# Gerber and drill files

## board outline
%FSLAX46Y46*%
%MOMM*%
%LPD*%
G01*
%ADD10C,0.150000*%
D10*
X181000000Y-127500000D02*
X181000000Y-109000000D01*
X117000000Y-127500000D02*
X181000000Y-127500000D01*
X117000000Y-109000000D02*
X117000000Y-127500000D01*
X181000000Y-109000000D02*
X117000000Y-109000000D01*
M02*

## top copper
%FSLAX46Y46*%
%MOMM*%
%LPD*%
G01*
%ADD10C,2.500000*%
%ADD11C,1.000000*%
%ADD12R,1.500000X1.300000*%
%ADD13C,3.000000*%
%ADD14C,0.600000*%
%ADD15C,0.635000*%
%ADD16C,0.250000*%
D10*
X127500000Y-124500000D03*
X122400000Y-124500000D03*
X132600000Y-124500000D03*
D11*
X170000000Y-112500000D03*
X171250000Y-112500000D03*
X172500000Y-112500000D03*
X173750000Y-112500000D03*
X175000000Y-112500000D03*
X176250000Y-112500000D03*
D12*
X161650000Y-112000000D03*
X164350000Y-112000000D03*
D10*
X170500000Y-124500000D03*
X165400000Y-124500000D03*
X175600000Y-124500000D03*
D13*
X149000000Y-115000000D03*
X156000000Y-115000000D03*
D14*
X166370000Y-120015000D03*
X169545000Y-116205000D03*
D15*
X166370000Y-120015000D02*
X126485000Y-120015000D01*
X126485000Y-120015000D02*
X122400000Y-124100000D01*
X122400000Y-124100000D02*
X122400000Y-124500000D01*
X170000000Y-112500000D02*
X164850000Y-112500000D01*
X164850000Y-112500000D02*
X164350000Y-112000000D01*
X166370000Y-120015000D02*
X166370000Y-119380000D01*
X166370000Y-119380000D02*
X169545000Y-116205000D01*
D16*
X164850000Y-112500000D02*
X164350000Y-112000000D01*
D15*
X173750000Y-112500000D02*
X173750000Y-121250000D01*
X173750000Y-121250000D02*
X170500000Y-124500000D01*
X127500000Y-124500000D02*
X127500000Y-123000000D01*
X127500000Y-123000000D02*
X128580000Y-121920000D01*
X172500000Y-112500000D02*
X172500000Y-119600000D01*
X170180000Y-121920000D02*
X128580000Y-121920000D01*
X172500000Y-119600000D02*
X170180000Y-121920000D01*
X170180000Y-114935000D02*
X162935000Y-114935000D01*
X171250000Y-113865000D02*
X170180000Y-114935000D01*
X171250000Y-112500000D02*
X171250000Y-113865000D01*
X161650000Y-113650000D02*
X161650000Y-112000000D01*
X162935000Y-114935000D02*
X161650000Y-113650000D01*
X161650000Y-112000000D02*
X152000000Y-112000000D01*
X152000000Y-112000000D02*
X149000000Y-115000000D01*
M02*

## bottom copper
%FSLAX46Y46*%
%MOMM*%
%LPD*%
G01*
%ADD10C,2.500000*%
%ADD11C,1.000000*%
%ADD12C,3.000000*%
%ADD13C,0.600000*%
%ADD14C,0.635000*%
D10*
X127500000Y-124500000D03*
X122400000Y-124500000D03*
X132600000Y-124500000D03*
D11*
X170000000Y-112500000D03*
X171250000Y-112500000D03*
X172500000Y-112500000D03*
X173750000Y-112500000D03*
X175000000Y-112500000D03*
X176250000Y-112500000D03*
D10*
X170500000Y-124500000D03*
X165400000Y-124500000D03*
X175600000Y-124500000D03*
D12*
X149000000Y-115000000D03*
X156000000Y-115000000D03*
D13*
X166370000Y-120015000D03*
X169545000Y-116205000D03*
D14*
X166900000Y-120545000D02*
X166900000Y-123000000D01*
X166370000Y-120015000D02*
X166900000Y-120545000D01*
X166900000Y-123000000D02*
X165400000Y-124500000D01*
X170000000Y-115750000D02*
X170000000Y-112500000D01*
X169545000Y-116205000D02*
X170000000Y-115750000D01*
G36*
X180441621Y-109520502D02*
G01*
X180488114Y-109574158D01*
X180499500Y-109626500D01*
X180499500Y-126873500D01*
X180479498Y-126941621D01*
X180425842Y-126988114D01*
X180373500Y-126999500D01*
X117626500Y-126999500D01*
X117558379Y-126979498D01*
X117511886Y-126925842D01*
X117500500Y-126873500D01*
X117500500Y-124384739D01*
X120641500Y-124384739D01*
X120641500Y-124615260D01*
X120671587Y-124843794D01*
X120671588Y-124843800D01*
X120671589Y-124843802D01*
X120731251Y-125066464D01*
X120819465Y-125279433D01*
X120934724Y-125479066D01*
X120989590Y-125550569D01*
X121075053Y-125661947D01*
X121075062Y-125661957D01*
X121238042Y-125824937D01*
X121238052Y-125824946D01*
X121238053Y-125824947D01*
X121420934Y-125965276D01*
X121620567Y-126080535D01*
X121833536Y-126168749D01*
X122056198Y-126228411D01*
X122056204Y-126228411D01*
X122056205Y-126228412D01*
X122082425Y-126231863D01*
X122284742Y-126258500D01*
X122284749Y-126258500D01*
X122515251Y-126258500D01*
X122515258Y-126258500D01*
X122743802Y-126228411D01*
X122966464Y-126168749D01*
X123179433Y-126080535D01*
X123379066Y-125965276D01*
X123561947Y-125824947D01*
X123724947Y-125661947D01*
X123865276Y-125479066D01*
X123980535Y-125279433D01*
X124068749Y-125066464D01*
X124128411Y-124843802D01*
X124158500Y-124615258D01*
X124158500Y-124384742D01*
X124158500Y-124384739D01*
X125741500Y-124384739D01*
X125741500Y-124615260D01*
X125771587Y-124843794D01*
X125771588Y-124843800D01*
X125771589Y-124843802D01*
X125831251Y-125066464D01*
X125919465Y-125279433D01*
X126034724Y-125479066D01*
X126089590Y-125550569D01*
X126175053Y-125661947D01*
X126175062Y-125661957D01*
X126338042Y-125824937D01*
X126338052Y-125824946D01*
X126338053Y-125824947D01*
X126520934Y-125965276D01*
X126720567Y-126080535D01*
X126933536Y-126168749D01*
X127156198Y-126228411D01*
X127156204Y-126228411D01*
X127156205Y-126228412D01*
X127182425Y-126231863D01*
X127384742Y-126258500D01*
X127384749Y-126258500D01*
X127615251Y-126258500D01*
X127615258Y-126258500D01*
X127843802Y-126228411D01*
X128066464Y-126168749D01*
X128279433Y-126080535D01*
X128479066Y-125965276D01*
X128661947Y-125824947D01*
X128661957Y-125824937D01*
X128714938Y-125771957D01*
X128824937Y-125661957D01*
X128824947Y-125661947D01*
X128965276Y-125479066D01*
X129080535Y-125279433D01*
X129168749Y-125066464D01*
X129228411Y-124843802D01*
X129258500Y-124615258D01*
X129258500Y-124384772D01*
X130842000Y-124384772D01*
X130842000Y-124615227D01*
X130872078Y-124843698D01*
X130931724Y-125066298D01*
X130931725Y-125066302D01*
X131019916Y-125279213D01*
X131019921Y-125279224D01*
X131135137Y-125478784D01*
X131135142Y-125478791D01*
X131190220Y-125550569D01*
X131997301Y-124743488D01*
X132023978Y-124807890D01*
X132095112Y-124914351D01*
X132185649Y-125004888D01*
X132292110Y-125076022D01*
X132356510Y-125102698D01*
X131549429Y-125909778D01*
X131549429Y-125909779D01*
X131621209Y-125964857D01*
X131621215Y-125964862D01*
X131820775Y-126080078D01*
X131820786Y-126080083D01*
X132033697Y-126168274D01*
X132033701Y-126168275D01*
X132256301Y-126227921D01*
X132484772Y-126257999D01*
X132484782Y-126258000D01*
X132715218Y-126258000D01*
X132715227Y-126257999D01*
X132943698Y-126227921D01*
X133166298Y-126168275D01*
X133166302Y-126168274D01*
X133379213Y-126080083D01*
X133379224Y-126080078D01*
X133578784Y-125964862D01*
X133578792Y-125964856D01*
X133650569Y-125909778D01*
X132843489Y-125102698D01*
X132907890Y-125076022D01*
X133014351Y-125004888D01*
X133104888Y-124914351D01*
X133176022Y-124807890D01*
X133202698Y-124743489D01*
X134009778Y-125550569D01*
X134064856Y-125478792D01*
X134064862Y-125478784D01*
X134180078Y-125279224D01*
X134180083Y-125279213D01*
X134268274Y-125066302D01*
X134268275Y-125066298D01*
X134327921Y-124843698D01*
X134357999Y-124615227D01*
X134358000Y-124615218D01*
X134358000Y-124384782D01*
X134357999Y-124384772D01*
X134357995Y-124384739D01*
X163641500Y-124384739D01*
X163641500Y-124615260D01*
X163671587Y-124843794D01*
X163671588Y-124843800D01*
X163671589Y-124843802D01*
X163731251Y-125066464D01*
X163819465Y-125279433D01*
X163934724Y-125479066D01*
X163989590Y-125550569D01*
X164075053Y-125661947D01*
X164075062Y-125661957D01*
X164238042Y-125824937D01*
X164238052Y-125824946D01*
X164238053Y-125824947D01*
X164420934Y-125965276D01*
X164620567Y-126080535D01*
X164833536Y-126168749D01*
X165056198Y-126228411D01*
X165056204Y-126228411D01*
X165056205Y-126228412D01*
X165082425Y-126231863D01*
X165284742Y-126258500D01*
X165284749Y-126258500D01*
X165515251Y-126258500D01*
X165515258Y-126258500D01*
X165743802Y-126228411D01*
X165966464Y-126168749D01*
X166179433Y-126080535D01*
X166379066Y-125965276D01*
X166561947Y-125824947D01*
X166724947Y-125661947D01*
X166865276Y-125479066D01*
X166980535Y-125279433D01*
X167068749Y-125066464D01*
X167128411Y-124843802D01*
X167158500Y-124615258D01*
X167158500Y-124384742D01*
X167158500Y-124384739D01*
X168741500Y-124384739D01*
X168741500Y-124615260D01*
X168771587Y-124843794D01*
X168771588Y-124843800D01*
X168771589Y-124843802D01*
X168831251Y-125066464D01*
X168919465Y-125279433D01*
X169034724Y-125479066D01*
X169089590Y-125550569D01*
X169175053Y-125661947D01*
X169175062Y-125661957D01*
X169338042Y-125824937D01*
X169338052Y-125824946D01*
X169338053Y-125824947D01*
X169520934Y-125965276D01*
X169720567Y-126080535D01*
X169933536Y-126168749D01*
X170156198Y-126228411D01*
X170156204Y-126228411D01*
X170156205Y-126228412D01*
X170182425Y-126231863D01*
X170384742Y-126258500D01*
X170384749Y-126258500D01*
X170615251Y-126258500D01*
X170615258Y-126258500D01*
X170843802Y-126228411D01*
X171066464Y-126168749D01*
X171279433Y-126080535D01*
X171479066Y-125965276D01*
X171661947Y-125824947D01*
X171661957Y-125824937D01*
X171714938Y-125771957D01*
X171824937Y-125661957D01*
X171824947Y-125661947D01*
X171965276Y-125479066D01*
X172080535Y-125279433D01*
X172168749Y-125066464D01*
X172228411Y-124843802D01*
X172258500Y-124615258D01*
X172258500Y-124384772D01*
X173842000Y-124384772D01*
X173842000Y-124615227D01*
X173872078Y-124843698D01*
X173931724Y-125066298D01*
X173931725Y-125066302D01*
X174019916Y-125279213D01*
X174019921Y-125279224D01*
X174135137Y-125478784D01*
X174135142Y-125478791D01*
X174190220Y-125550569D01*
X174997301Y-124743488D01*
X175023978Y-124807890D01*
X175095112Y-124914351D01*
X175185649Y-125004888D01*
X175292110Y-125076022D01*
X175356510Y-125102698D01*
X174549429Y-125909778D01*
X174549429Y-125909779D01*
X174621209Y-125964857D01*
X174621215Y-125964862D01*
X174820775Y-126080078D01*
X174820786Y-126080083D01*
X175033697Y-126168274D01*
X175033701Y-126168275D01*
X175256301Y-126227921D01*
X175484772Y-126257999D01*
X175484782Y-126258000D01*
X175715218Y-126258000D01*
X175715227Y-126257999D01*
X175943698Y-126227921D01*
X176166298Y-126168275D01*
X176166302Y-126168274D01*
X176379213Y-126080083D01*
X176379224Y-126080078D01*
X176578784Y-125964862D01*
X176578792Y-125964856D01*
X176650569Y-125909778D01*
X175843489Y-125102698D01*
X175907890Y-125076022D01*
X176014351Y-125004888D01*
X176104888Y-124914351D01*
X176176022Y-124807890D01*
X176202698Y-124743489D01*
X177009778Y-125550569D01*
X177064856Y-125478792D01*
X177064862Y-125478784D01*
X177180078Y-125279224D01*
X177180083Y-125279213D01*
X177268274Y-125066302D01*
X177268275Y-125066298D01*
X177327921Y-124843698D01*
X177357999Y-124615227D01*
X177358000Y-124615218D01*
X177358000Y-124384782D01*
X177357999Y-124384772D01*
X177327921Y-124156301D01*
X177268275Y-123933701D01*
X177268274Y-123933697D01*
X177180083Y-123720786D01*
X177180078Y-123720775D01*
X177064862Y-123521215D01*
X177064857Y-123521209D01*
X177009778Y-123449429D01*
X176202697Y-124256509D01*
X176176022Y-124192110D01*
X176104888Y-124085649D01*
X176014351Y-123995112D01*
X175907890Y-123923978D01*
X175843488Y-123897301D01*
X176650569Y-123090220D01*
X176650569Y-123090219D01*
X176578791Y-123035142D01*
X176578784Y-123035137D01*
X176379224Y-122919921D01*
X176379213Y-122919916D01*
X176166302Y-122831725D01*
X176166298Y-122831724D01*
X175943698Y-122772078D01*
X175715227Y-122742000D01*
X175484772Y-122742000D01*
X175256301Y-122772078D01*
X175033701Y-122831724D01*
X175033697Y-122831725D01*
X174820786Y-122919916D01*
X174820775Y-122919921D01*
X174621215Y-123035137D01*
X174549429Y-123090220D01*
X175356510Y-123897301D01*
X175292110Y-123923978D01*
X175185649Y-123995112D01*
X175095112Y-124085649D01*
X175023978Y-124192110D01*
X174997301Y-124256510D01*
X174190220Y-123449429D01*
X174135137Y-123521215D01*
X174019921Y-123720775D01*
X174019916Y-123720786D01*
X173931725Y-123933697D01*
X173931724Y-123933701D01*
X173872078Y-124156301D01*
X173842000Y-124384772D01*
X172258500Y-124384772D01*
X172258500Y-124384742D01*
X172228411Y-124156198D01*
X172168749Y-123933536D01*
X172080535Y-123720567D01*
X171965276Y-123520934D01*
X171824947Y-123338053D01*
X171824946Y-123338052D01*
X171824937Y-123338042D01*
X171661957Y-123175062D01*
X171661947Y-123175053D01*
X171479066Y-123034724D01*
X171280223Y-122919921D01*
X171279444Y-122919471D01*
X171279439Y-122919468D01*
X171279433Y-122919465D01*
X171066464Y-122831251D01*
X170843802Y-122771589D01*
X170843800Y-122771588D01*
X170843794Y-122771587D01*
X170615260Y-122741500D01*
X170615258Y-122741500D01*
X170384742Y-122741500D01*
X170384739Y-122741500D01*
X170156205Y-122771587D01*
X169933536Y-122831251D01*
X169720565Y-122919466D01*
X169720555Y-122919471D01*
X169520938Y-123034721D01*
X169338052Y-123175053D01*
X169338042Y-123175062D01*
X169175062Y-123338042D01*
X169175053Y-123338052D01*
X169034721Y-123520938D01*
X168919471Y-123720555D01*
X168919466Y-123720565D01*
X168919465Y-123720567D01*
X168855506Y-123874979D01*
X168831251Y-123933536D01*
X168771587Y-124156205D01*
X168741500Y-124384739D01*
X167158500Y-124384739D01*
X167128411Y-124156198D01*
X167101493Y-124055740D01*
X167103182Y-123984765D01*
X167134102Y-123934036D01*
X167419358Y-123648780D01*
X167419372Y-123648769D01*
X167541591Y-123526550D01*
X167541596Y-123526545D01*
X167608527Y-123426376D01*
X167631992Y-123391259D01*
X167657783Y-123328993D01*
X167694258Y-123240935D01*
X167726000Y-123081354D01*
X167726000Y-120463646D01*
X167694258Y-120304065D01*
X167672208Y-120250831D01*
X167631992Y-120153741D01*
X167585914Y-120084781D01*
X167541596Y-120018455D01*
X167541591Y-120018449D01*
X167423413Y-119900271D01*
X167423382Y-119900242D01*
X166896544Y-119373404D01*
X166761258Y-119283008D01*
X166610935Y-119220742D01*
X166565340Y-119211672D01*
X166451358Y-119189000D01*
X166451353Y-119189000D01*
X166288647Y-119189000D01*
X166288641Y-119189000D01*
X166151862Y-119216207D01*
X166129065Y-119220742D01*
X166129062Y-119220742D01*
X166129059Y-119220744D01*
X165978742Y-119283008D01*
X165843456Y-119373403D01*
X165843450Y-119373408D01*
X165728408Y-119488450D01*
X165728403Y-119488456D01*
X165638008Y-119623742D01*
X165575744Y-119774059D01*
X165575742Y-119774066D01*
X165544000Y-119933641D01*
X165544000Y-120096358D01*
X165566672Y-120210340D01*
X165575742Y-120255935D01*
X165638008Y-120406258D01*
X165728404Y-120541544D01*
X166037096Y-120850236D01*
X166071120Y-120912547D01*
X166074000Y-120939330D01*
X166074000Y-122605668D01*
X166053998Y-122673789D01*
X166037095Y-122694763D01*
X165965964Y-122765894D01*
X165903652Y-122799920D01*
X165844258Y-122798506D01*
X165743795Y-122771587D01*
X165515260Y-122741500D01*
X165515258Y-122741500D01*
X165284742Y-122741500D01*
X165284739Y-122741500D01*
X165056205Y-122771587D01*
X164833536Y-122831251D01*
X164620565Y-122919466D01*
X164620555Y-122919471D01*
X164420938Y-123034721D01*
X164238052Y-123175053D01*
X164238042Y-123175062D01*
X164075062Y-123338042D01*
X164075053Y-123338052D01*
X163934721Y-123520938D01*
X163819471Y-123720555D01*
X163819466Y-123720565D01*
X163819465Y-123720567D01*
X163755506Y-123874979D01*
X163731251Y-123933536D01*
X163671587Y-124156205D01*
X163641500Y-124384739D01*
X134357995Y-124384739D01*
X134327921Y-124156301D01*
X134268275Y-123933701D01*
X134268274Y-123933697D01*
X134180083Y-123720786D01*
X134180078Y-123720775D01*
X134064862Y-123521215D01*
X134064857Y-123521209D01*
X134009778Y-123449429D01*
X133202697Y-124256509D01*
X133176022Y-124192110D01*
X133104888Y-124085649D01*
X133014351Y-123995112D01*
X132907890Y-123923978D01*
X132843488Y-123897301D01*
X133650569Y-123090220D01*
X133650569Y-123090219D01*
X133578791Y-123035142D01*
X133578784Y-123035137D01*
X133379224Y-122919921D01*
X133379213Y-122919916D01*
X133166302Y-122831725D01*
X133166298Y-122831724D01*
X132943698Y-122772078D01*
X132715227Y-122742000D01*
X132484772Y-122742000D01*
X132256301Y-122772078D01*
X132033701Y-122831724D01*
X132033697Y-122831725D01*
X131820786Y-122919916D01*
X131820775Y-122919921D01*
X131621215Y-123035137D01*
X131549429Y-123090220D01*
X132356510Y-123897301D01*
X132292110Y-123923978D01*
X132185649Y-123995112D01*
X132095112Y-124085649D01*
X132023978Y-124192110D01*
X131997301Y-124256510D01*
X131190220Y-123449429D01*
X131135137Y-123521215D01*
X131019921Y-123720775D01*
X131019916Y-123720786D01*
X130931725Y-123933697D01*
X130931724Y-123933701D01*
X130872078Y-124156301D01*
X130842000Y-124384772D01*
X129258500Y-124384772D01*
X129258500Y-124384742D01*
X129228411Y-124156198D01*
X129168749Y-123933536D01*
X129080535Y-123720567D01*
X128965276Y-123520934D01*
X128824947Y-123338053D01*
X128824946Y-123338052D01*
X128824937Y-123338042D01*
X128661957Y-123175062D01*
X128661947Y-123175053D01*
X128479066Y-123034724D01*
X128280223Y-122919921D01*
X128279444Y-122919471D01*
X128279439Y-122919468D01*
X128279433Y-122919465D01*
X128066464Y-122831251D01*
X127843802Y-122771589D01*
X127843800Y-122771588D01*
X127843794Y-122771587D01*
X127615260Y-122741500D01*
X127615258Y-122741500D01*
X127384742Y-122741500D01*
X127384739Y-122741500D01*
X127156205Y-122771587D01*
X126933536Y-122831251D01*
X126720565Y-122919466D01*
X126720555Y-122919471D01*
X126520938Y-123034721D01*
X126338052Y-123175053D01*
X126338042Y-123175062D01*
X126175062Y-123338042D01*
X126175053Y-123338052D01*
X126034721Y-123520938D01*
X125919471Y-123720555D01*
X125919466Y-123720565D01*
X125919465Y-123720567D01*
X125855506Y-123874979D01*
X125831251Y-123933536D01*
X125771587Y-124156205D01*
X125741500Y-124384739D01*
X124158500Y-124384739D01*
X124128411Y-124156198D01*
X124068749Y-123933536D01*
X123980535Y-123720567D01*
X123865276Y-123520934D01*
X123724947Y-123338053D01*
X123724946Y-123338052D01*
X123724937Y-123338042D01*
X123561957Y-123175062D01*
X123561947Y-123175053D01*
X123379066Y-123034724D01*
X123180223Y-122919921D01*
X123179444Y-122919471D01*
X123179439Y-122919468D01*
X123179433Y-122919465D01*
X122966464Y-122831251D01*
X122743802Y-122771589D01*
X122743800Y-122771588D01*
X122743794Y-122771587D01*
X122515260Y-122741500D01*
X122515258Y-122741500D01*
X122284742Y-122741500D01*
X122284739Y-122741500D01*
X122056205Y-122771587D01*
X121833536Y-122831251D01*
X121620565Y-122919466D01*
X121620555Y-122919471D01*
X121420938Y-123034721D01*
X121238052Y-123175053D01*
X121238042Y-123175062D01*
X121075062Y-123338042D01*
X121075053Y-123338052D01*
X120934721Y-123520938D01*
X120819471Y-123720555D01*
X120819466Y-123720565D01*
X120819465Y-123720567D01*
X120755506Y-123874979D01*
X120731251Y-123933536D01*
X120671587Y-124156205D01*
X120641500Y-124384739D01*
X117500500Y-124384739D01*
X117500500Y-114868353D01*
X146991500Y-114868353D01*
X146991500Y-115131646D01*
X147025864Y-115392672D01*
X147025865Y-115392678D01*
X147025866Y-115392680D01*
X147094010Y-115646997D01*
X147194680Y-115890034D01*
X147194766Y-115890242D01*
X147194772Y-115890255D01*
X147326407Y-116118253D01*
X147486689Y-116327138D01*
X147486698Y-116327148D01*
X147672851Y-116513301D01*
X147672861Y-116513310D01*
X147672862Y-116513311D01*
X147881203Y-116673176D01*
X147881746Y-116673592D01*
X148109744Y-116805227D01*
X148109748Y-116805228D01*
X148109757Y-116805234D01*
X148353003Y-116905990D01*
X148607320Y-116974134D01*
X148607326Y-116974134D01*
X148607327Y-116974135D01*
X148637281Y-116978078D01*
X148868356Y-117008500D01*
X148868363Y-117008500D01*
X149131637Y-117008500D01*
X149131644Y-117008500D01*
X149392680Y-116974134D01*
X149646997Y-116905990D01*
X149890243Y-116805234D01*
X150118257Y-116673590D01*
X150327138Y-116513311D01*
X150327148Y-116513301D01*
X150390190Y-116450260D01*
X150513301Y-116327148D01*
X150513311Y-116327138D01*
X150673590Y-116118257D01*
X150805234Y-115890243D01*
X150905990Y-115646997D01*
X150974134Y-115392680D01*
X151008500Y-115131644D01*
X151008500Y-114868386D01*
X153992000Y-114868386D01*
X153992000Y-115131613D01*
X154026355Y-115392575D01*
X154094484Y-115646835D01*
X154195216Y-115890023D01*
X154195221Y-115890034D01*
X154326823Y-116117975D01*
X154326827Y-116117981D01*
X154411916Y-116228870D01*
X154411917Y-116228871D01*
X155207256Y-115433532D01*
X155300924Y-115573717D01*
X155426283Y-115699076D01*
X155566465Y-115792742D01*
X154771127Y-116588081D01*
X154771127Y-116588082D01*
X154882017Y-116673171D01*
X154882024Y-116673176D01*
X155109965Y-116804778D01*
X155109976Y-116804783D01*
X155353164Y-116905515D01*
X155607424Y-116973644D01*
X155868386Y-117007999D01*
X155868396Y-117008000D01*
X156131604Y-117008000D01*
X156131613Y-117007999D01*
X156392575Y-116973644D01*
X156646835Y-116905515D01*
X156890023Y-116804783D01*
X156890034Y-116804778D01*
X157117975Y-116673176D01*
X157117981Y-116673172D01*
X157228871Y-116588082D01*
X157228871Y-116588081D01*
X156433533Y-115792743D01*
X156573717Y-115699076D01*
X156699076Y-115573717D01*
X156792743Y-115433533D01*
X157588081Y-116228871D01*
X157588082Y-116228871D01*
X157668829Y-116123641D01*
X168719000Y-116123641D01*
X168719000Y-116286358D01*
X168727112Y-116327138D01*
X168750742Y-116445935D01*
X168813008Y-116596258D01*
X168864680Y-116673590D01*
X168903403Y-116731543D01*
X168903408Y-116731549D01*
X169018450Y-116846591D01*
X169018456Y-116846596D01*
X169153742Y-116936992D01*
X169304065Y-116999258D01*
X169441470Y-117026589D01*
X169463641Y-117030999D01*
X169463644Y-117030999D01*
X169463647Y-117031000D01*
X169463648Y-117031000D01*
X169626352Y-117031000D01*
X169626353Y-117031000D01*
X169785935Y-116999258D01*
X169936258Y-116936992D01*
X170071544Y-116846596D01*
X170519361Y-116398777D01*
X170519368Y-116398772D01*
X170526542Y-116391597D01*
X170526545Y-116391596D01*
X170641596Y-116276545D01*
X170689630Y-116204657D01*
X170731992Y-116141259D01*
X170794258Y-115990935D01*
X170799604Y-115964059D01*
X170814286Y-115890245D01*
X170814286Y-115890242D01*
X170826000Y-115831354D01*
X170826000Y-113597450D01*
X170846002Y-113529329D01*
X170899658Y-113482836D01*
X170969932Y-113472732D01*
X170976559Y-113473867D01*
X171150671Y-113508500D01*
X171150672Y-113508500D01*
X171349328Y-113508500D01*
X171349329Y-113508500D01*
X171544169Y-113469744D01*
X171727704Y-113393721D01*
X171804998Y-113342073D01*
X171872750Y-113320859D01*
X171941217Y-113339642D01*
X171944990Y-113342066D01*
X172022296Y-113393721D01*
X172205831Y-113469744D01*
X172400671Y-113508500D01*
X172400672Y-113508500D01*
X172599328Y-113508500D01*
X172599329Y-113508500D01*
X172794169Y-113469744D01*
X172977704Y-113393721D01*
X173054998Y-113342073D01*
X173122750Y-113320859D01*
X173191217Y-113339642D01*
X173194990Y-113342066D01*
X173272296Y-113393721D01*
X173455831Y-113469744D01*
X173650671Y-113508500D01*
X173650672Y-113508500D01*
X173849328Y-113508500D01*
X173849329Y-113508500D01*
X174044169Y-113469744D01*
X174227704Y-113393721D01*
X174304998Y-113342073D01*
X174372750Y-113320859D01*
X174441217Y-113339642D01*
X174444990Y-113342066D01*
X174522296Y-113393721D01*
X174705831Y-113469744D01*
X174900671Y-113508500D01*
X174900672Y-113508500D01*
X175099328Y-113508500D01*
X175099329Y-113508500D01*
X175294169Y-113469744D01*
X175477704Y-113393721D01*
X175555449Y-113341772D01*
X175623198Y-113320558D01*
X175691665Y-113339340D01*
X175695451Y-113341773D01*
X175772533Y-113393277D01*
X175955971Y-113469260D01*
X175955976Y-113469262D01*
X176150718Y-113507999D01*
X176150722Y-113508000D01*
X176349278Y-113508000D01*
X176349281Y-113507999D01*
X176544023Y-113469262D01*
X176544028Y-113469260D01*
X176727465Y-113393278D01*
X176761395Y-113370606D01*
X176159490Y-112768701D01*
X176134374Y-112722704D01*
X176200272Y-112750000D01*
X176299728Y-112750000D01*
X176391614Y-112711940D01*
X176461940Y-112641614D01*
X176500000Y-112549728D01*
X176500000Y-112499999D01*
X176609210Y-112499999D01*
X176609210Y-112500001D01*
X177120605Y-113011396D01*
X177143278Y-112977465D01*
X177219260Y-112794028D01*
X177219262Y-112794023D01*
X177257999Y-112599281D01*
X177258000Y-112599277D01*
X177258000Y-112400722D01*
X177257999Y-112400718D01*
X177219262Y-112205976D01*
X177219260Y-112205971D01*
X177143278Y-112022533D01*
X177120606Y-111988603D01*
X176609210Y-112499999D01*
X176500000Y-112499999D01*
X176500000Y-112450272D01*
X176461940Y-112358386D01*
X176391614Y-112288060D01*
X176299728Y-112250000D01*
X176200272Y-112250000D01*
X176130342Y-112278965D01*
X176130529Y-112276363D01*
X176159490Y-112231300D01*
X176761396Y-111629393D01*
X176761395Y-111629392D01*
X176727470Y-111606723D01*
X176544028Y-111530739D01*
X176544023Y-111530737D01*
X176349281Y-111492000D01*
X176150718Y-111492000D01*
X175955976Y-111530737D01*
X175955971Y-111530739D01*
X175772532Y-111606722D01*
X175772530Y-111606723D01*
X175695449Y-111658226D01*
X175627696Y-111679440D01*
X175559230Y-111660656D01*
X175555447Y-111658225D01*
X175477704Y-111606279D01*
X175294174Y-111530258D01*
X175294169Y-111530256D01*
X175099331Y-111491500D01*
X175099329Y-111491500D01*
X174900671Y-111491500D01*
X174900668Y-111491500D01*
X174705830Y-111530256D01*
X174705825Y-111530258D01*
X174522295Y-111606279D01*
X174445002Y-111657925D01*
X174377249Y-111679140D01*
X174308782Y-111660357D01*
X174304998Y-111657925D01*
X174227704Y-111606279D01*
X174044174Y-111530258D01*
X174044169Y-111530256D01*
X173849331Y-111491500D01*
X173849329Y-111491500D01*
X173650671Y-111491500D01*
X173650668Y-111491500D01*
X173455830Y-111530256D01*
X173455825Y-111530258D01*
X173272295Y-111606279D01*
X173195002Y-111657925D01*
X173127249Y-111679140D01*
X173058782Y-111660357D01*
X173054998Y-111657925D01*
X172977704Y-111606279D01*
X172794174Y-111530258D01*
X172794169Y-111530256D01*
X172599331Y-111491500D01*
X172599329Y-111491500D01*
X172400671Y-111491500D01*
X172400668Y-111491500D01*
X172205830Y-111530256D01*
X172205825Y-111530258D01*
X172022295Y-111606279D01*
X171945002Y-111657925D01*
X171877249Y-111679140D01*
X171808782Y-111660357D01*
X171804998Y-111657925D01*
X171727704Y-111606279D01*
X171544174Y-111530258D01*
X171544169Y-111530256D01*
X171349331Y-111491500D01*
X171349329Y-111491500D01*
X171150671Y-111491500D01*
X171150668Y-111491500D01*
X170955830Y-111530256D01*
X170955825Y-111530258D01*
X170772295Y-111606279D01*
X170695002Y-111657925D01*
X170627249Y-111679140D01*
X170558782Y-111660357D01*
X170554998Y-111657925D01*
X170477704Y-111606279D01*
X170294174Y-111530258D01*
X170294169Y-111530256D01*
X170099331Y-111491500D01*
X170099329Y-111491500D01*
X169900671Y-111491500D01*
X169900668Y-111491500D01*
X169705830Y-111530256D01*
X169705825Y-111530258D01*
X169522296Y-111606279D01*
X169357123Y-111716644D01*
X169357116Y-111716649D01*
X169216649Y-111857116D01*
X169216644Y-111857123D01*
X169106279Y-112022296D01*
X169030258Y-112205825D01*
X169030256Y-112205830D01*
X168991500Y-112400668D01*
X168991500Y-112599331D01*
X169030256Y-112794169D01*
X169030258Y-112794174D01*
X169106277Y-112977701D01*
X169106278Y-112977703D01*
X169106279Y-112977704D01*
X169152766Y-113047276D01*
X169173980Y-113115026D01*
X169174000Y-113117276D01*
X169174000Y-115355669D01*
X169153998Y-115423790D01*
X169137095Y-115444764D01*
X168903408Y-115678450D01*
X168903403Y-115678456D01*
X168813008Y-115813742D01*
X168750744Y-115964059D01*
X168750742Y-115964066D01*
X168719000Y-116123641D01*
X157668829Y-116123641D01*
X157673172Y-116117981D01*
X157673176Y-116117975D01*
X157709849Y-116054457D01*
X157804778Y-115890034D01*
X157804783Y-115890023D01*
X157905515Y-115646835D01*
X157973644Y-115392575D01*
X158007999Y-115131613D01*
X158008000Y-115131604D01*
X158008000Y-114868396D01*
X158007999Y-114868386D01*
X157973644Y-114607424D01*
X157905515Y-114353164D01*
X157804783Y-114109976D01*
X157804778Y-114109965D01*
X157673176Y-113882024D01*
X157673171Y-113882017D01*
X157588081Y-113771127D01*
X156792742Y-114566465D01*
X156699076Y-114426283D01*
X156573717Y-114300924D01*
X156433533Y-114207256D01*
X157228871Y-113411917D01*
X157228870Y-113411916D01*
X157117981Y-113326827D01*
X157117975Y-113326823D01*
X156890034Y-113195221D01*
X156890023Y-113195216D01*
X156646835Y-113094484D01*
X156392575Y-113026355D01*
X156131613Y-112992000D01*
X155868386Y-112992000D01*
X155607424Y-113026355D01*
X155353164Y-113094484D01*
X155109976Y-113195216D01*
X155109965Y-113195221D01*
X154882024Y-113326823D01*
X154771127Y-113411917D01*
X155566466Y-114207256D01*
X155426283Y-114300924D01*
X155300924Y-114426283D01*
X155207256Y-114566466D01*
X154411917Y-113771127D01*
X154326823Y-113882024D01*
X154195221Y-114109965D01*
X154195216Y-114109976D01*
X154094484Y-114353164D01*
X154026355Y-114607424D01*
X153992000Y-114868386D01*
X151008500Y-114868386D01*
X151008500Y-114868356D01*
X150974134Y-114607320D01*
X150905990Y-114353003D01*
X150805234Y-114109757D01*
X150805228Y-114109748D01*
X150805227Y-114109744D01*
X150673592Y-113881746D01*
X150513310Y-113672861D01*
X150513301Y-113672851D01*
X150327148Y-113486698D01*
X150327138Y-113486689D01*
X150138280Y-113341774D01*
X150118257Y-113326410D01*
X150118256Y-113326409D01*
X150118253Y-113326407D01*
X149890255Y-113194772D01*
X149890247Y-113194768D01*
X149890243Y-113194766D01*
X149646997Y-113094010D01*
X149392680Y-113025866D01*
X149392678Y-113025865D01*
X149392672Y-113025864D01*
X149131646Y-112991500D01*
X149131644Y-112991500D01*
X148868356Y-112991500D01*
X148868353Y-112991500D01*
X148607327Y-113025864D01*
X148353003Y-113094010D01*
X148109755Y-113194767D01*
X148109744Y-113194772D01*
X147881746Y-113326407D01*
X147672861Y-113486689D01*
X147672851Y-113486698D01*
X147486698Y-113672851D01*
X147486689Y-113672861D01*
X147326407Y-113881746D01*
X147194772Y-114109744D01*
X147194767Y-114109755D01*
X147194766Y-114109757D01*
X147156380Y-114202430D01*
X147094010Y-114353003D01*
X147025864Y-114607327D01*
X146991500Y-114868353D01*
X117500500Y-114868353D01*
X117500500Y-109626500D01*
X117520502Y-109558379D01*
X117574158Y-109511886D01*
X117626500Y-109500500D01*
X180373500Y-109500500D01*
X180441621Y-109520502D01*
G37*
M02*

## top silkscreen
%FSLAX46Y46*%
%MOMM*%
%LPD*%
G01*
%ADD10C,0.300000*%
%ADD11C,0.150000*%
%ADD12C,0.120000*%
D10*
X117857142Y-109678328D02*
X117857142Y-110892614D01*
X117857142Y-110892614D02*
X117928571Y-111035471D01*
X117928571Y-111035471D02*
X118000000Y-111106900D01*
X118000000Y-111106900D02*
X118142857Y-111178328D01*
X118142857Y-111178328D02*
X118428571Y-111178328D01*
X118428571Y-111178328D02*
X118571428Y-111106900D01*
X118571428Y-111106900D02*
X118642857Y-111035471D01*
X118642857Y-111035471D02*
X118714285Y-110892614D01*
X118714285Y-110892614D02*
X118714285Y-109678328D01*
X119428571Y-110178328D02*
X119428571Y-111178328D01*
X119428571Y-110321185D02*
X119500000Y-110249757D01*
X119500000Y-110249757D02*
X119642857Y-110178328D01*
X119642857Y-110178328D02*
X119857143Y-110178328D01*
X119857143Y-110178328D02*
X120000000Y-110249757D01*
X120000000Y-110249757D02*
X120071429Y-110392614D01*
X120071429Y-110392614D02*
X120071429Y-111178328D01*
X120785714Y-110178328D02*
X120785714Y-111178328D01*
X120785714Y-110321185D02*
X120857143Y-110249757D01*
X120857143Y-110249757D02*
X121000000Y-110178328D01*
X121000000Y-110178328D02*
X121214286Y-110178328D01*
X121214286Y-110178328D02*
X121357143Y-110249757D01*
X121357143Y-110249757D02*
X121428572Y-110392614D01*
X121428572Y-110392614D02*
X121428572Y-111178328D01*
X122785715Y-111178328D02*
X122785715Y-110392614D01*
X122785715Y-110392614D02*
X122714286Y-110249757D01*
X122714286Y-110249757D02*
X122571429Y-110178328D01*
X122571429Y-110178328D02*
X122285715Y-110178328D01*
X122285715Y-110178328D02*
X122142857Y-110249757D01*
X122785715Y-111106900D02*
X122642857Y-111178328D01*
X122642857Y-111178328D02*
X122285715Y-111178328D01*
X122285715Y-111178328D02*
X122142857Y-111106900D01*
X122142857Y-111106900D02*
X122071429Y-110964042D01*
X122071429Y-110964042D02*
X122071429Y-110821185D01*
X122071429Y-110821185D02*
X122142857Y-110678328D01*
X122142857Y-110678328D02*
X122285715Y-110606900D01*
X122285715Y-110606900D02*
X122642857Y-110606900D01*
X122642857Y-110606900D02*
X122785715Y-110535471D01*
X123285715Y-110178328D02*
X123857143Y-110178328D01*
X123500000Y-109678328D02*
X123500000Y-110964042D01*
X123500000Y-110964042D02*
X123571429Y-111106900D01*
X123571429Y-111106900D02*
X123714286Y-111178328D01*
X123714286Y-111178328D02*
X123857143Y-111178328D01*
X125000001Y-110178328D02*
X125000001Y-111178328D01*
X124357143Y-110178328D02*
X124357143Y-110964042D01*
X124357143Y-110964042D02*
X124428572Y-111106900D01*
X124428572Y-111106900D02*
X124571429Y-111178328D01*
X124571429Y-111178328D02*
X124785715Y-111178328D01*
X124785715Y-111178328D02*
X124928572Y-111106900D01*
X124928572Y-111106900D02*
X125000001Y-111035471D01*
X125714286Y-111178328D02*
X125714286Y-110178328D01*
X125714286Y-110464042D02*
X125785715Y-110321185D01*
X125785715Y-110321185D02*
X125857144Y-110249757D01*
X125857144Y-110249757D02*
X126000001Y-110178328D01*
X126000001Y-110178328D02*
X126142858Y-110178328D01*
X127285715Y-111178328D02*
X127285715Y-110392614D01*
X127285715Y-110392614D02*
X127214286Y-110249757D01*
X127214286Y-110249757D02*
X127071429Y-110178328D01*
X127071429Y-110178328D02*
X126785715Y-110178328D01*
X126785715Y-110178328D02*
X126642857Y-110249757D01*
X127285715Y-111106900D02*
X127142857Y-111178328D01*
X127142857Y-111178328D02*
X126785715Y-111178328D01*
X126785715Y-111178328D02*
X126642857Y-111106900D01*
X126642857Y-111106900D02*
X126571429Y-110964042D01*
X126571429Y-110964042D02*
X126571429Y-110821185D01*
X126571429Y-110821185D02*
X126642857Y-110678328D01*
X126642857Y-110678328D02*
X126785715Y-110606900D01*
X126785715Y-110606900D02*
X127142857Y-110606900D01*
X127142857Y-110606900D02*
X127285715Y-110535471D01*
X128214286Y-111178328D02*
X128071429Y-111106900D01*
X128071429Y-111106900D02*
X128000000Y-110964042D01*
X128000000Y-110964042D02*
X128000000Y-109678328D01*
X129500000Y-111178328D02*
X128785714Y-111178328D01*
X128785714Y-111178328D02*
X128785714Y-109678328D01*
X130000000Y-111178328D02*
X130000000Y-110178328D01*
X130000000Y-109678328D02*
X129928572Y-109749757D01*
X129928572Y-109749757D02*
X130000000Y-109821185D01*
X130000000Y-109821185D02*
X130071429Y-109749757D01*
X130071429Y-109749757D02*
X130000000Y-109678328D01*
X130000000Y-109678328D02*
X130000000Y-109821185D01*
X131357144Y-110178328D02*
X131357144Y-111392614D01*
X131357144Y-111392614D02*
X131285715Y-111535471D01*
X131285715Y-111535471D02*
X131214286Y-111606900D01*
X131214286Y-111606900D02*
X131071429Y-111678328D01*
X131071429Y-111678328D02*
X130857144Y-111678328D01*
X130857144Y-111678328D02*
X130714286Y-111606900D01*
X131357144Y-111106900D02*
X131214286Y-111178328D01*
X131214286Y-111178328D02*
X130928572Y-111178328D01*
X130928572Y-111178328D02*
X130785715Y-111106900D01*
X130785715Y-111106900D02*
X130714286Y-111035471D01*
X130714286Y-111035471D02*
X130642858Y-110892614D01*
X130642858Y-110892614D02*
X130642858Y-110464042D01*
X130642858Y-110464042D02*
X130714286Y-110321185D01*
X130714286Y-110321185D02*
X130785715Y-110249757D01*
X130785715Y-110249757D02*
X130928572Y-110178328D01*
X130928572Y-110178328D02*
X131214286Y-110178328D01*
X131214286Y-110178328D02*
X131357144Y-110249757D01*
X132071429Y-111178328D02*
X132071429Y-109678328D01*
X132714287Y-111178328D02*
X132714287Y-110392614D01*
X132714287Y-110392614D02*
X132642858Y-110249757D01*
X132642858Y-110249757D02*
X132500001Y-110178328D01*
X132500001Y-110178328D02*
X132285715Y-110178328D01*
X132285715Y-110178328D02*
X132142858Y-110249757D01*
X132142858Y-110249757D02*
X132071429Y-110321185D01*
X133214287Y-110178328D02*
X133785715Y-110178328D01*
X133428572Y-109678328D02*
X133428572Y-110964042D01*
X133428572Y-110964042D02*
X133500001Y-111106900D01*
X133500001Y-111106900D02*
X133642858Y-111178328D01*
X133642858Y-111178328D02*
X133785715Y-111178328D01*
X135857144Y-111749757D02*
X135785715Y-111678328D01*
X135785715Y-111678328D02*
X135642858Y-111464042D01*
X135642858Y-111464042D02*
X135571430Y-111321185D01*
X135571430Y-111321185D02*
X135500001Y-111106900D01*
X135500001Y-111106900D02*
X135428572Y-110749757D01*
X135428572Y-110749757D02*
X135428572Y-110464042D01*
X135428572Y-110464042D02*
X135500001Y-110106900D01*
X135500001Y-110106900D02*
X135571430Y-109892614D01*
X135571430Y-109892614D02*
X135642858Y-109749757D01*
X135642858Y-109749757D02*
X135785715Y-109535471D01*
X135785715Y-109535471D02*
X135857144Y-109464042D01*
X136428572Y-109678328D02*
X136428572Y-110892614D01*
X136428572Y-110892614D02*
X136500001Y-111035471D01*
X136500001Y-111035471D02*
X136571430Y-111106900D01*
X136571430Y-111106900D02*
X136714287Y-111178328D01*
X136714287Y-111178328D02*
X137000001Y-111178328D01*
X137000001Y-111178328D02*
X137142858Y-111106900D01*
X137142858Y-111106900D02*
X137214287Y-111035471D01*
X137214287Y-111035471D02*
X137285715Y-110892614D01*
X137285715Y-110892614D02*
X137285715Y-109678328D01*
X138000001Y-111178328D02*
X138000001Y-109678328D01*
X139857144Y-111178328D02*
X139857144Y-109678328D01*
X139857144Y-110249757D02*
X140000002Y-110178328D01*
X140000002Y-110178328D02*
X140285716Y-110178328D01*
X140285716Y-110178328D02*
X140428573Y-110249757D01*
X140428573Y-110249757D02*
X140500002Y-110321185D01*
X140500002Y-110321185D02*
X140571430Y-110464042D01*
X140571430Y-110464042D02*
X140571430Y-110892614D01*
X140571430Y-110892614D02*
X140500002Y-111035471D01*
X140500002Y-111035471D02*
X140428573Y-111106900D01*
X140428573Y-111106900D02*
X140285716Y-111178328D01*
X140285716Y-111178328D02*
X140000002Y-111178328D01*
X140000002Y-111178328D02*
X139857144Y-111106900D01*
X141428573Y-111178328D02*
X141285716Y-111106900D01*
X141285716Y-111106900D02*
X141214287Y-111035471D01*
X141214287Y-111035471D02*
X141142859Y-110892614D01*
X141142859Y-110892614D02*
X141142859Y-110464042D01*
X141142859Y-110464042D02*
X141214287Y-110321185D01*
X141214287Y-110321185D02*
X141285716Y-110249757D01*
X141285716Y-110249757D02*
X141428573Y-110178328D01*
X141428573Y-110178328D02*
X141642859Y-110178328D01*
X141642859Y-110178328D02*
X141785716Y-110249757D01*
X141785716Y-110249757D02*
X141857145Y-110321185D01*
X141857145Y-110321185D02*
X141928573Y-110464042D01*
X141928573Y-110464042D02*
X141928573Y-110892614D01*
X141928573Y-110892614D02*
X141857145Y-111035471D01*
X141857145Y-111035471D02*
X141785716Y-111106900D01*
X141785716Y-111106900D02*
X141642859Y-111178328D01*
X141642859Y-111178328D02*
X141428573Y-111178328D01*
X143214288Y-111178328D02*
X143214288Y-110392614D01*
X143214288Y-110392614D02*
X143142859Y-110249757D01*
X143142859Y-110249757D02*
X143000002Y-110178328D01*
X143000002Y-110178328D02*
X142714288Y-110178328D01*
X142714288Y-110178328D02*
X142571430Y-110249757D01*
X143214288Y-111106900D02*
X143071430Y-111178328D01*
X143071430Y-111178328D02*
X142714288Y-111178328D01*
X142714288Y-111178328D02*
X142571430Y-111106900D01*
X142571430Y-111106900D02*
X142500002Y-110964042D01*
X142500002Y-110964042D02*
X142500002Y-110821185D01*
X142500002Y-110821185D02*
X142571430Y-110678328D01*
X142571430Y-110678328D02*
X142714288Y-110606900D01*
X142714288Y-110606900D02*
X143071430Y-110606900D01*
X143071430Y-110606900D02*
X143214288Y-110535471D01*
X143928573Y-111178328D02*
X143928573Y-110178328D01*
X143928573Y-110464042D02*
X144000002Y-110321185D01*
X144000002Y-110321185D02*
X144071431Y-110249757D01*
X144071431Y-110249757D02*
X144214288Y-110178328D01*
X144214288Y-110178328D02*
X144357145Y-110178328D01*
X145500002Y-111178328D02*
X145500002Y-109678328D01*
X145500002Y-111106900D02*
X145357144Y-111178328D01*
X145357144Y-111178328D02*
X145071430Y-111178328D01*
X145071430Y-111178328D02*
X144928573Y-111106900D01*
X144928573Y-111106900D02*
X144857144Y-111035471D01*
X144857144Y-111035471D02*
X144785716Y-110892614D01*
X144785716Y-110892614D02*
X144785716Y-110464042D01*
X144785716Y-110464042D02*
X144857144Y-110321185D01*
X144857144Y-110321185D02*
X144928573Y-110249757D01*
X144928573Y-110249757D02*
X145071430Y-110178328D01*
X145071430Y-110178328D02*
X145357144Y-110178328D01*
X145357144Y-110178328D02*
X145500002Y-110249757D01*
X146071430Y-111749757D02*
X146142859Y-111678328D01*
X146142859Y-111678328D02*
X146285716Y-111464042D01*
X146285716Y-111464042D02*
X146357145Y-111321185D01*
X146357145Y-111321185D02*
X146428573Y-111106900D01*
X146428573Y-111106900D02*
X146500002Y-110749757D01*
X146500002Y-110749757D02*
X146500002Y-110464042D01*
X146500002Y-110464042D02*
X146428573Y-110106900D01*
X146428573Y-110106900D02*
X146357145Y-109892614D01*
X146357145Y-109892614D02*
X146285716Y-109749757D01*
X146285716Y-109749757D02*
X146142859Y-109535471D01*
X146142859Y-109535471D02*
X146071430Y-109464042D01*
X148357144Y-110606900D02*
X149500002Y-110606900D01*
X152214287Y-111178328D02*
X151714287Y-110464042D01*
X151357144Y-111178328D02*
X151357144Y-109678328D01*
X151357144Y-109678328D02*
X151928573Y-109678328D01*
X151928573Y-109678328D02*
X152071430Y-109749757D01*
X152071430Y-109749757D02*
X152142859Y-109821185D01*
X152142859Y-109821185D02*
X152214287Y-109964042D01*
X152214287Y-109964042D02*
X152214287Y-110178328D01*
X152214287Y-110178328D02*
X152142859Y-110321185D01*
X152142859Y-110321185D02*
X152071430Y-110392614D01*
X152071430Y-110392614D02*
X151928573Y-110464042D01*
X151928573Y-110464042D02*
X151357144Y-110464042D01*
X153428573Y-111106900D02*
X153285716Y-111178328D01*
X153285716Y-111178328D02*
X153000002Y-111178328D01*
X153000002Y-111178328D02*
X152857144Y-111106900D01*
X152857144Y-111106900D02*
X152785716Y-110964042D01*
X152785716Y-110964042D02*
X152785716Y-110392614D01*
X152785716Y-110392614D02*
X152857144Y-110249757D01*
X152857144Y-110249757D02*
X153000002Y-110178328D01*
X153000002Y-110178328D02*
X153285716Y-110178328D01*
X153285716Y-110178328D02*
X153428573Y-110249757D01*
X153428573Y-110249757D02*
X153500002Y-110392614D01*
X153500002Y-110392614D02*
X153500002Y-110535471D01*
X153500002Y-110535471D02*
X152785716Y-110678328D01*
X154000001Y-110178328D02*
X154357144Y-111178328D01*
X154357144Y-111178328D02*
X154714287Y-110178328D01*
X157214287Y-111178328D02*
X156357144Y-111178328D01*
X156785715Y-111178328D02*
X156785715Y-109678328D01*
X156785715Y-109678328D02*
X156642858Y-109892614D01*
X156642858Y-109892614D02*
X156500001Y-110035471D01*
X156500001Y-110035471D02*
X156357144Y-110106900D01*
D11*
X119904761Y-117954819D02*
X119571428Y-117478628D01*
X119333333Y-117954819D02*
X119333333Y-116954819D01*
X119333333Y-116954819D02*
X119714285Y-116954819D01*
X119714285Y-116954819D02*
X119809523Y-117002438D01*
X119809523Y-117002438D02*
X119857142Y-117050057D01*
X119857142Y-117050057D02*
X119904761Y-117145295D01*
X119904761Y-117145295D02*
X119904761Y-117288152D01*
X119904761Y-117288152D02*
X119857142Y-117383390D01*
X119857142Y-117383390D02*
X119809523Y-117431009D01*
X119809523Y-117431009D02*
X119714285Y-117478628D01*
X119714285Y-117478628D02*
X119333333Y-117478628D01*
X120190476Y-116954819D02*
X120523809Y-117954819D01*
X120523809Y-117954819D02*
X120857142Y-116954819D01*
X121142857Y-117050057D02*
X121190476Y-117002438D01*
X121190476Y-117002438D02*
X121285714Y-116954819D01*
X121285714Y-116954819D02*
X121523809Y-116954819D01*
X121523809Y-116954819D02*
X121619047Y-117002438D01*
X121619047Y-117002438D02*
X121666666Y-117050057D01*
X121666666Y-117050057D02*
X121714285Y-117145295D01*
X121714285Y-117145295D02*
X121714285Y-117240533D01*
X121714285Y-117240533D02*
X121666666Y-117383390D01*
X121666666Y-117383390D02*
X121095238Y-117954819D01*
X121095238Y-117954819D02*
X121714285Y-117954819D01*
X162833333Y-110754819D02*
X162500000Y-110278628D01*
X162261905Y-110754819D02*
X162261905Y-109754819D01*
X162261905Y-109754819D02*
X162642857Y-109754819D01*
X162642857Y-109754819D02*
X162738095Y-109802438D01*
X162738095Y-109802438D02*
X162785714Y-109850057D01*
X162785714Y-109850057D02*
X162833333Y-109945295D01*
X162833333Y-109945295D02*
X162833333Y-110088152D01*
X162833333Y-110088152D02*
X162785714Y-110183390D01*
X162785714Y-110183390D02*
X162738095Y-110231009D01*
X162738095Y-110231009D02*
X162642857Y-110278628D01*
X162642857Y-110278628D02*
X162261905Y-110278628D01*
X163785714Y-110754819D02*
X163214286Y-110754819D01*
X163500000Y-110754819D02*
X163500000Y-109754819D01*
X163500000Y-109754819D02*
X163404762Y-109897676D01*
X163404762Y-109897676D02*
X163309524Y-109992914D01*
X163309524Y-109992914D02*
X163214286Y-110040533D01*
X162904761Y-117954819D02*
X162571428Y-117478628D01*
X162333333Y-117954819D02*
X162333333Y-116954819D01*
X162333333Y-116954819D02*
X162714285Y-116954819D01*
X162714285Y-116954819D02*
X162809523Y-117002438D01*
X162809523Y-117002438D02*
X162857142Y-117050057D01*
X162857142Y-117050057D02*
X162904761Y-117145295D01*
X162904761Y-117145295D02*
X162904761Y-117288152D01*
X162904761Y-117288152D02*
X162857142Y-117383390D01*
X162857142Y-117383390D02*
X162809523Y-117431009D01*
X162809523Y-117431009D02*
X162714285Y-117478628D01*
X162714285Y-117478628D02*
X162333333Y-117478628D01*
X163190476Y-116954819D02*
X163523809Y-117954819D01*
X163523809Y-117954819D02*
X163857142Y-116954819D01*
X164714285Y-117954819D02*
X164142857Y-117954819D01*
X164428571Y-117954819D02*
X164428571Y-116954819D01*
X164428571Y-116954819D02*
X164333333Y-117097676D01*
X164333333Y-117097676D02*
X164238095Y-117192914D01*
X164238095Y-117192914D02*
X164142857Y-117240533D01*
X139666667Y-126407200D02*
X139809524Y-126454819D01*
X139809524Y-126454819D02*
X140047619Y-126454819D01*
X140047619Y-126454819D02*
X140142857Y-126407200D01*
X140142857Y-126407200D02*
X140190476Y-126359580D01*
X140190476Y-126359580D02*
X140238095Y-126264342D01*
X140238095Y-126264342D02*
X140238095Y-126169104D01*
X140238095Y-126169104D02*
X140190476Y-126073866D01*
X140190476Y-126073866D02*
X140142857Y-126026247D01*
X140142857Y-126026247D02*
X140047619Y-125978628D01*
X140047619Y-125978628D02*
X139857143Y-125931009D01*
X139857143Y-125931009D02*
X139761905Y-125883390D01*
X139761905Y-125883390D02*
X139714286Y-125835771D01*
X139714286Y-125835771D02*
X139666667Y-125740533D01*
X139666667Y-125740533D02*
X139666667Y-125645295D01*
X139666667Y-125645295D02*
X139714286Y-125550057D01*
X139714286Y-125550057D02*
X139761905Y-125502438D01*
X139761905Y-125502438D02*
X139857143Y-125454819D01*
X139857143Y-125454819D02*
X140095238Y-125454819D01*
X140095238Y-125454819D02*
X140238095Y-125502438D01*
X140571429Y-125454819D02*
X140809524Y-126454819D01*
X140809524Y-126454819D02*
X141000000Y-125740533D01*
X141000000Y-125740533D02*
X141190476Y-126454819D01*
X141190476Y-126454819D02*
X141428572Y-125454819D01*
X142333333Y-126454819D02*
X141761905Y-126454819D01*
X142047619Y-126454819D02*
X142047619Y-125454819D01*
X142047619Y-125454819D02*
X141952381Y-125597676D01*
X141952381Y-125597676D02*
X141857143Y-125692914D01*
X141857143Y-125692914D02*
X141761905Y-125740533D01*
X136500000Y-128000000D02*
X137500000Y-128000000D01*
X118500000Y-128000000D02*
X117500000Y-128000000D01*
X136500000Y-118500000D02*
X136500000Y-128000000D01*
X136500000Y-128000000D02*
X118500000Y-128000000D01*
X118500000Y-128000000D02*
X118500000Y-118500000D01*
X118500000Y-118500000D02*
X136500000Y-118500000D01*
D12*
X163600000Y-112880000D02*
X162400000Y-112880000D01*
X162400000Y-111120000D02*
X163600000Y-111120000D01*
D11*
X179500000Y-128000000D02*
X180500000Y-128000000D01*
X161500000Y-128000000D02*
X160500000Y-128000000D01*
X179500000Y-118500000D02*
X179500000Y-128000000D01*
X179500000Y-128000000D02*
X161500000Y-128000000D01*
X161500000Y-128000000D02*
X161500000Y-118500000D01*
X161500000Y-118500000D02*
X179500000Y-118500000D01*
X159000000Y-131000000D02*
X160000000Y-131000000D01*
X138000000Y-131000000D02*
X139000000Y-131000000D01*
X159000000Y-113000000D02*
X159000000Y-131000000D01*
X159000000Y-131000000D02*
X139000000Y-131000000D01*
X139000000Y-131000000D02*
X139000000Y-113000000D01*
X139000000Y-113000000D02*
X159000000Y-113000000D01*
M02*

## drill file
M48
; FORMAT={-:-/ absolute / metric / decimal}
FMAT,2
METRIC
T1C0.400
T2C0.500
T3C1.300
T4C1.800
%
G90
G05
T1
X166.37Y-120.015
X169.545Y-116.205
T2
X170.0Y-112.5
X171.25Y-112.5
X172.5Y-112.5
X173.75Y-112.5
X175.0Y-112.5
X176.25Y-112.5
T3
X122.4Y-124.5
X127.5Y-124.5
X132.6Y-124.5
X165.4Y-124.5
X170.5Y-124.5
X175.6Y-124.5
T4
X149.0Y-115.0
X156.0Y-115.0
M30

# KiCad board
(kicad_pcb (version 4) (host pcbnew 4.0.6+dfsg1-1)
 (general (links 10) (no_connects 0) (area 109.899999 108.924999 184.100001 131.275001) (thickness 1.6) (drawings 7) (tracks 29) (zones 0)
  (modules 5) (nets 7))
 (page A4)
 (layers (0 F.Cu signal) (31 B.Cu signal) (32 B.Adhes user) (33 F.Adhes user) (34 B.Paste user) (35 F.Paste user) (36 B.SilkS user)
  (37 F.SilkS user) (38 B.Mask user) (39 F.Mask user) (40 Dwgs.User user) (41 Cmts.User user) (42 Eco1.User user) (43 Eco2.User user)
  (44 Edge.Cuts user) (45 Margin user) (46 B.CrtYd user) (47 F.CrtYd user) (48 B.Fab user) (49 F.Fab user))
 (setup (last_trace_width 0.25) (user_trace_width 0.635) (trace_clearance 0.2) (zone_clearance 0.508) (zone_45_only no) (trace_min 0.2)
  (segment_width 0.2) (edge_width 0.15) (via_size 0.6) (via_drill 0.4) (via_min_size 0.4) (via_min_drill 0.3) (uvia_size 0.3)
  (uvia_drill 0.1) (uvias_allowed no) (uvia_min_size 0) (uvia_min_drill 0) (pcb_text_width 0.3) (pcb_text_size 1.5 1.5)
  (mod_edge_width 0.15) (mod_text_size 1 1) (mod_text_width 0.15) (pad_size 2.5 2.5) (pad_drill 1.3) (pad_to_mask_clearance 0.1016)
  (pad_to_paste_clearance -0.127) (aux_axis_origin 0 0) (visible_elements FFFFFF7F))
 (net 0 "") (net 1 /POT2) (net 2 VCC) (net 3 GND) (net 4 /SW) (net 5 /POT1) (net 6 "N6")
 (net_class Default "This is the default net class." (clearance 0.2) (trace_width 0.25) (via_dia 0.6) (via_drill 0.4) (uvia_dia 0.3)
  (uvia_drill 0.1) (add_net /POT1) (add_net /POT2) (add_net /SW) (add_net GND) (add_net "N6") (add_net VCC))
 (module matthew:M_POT (layer F.Cu) (at 127.5 124.5)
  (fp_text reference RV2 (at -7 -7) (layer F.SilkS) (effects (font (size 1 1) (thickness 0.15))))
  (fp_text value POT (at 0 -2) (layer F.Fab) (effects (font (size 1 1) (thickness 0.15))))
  (fp_line (start 9 3.5) (end 10 3.5) (layer F.SilkS) (width 0.15))
  (fp_line (start -9 3.5) (end -10 3.5) (layer F.SilkS) (width 0.15))
  (fp_line (start 9 -6) (end 9 3.5) (layer F.SilkS) (width 0.15))
  (fp_line (start 9 3.5) (end -9 3.5) (layer F.SilkS) (width 0.15))
  (fp_line (start -9 3.5) (end -9 -6) (layer F.SilkS) (width 0.15))
  (fp_line (start -9 -6) (end 9 -6) (layer F.SilkS) (width 0.15))
  (pad 2 thru_hole circle (at 0 0) (size 2.5 2.5) (drill 1.3) (layers *.Cu *.Mask) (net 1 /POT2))
  (pad 1 thru_hole circle (at -5.1 0) (size 2.5 2.5) (drill 1.3) (layers *.Cu *.Mask) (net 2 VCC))
  (pad 3 thru_hole circle (at 5.1 0) (size 2.5 2.5) (drill 1.3) (layers *.Cu *.Mask) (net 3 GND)))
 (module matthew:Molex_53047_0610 (layer B.Cu) (at 170 112.5)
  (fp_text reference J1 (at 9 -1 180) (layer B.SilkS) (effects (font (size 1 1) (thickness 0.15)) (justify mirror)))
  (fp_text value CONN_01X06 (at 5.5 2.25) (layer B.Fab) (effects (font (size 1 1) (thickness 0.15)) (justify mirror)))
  (pad 1 thru_hole circle (at 0 0) (size 1 1) (drill 0.5) (layers *.Cu *.Mask) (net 2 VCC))
  (pad 2 thru_hole circle (at 1.25 0) (size 1 1) (drill 0.5) (layers *.Cu *.Mask) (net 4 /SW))
  (pad 3 thru_hole circle (at 2.5 0) (size 1 1) (drill 0.5) (layers *.Cu *.Mask) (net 1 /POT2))
  (pad 4 thru_hole circle (at 3.75 0) (size 1 1) (drill 0.5) (layers *.Cu *.Mask) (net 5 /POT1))
  (pad 5 thru_hole circle (at 5 0) (size 1 1) (drill 0.5) (layers *.Cu *.Mask) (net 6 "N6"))
  (pad 6 thru_hole circle (at 6.25 0) (size 1 1) (drill 0.5) (layers *.Cu *.Mask) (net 3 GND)))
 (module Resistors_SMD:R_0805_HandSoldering (layer F.Cu) (at 163 112)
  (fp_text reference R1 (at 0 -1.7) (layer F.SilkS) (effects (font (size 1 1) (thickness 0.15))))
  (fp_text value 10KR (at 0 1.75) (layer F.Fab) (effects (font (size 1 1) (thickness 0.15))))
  (fp_line (start 0.6 0.88) (end -0.6 0.88) (layer F.SilkS) (width 0.12))
  (fp_line (start -0.6 -0.88) (end 0.6 -0.88) (layer F.SilkS) (width 0.12))
  (pad 1 smd rect (at -1.35 0) (size 1.5 1.3) (layers F.Cu F.Paste F.Mask) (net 4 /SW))
  (pad 2 smd rect (at 1.35 0) (size 1.5 1.3) (layers F.Cu F.Paste F.Mask) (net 2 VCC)))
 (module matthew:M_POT (layer F.Cu) (at 170.5 124.5)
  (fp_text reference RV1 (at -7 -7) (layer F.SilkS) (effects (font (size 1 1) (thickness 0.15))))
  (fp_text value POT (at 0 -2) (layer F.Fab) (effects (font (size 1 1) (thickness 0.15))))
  (fp_line (start 9 3.5) (end 10 3.5) (layer F.SilkS) (width 0.15))
  (fp_line (start -9 3.5) (end -10 3.5) (layer F.SilkS) (width 0.15))
  (fp_line (start 9 -6) (end 9 3.5) (layer F.SilkS) (width 0.15))
  (fp_line (start 9 3.5) (end -9 3.5) (layer F.SilkS) (width 0.15))
  (fp_line (start -9 3.5) (end -9 -6) (layer F.SilkS) (width 0.15))
  (fp_line (start -9 -6) (end 9 -6) (layer F.SilkS) (width 0.15))
  (pad 2 thru_hole circle (at 0 0) (size 2.5 2.5) (drill 1.3) (layers *.Cu *.Mask) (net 5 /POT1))
  (pad 1 thru_hole circle (at -5.1 0) (size 2.5 2.5) (drill 1.3) (layers *.Cu *.Mask) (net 2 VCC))
  (pad 3 thru_hole circle (at 5.1 0) (size 2.5 2.5) (drill 1.3) (layers *.Cu *.Mask) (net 3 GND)))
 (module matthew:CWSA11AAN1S (layer F.Cu) (at 149 115)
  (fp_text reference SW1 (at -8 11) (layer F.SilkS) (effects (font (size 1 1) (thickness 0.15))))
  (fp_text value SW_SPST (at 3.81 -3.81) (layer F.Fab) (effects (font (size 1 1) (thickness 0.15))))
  (fp_line (start 10 16) (end 11 16) (layer F.SilkS) (width 0.15))
  (fp_line (start -11 16) (end -10 16) (layer F.SilkS) (width 0.15))
  (fp_line (start 10 -2) (end 10 16) (layer F.SilkS) (width 0.15))
  (fp_line (start 10 16) (end -10 16) (layer F.SilkS) (width 0.15))
  (fp_line (start -10 16) (end -10 -2) (layer F.SilkS) (width 0.15))
  (fp_line (start -10 -2) (end 10 -2) (layer F.SilkS) (width 0.15))
  (pad 1 thru_hole circle (at 0 0) (size 3 3) (drill 1.8) (layers *.Cu *.Mask) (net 4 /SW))
  (pad 2 thru_hole circle (at 7 0) (size 3 3) (drill 1.8) (layers *.Cu *.Mask) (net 3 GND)))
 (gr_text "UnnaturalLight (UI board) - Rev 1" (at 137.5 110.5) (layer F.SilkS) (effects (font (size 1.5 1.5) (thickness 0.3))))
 (gr_line (start 181 127.5) (end 181 109) (angle 90) (layer Edge.Cuts) (width 0.15))
 (gr_line (start 117 127.5) (end 181 127.5) (angle 90) (layer Edge.Cuts) (width 0.15))
 (gr_line (start 117 109) (end 117 127.5) (angle 90) (layer Edge.Cuts) (width 0.15))
 (gr_line (start 181 109) (end 117 109) (angle 90) (layer Edge.Cuts) (width 0.15))
 (segment (start 166.37 120.015) (end 126.485 120.015) (width 0.635) (layer F.Cu) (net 2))
 (segment (start 126.485 120.015) (end 122.4 124.1) (width 0.635) (layer F.Cu) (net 2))
 (segment (start 122.4 124.1) (end 122.4 124.5) (width 0.635) (layer F.Cu) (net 2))
 (segment (start 166.9 120.545) (end 166.9 123) (width 0.635) (layer B.Cu) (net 2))
 (segment (start 166.37 120.015) (end 166.9 120.545) (width 0.635) (layer B.Cu) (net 2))
 (via (at 166.37 120.015) (size 0.6) (drill 0.4) (layers F.Cu B.Cu) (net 2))
 (segment (start 166.9 123) (end 165.4 124.5) (width 0.635) (layer B.Cu) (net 2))
 (segment (start 170 112.5) (end 164.85 112.5) (width 0.635) (layer F.Cu) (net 2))
 (segment (start 164.85 112.5) (end 164.35 112) (width 0.635) (layer F.Cu) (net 2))
 (segment (start 166.37 120.015) (end 166.37 119.38) (width 0.635) (layer F.Cu) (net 2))
 (segment (start 170 115.75) (end 170 112.5) (width 0.635) (layer B.Cu) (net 2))
 (segment (start 169.545 116.205) (end 170 115.75) (width 0.635) (layer B.Cu) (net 2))
 (via (at 169.545 116.205) (size 0.6) (drill 0.4) (layers F.Cu B.Cu) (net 2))
 (segment (start 166.37 119.38) (end 169.545 116.205) (width 0.635) (layer F.Cu) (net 2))
 (segment (start 164.85 112.5) (end 164.35 112) (width 0.25) (layer F.Cu) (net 2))
 (segment (start 173.75 112.5) (end 173.75 121.25) (width 0.635) (layer F.Cu) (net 5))
 (segment (start 173.75 121.25) (end 170.5 124.5) (width 0.635) (layer F.Cu) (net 5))
 (segment (start 127.5 124.5) (end 127.5 123) (width 0.635) (layer F.Cu) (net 1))
 (segment (start 127.5 123) (end 128.58 121.92) (width 0.635) (layer F.Cu) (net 1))
 (segment (start 172.5 112.5) (end 172.5 119.6) (width 0.635) (layer F.Cu) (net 1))
 (segment (start 170.18 121.92) (end 128.58 121.92) (width 0.635) (layer F.Cu) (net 1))
 (segment (start 172.5 119.6) (end 170.18 121.92) (width 0.635) (layer F.Cu) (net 1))
 (segment (start 170.18 114.935) (end 162.935 114.935) (width 0.635) (layer F.Cu) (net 4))
 (segment (start 171.25 113.865) (end 170.18 114.935) (width 0.635) (layer F.Cu) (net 4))
 (segment (start 171.25 112.5) (end 171.25 113.865) (width 0.635) (layer F.Cu) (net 4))
 (segment (start 161.65 113.65) (end 161.65 112) (width 0.635) (layer F.Cu) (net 4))
 (segment (start 162.935 114.935) (end 161.65 113.65) (width 0.635) (layer F.Cu) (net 4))
 (segment (start 161.65 112) (end 152 112) (width 0.635) (layer F.Cu) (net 4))
 (segment (start 152 112) (end 149 115) (width 0.635) (layer F.Cu) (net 4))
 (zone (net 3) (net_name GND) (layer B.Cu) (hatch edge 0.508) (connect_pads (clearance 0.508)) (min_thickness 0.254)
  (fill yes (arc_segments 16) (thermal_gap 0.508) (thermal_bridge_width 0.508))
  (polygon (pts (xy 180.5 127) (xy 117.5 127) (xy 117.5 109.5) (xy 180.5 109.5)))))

